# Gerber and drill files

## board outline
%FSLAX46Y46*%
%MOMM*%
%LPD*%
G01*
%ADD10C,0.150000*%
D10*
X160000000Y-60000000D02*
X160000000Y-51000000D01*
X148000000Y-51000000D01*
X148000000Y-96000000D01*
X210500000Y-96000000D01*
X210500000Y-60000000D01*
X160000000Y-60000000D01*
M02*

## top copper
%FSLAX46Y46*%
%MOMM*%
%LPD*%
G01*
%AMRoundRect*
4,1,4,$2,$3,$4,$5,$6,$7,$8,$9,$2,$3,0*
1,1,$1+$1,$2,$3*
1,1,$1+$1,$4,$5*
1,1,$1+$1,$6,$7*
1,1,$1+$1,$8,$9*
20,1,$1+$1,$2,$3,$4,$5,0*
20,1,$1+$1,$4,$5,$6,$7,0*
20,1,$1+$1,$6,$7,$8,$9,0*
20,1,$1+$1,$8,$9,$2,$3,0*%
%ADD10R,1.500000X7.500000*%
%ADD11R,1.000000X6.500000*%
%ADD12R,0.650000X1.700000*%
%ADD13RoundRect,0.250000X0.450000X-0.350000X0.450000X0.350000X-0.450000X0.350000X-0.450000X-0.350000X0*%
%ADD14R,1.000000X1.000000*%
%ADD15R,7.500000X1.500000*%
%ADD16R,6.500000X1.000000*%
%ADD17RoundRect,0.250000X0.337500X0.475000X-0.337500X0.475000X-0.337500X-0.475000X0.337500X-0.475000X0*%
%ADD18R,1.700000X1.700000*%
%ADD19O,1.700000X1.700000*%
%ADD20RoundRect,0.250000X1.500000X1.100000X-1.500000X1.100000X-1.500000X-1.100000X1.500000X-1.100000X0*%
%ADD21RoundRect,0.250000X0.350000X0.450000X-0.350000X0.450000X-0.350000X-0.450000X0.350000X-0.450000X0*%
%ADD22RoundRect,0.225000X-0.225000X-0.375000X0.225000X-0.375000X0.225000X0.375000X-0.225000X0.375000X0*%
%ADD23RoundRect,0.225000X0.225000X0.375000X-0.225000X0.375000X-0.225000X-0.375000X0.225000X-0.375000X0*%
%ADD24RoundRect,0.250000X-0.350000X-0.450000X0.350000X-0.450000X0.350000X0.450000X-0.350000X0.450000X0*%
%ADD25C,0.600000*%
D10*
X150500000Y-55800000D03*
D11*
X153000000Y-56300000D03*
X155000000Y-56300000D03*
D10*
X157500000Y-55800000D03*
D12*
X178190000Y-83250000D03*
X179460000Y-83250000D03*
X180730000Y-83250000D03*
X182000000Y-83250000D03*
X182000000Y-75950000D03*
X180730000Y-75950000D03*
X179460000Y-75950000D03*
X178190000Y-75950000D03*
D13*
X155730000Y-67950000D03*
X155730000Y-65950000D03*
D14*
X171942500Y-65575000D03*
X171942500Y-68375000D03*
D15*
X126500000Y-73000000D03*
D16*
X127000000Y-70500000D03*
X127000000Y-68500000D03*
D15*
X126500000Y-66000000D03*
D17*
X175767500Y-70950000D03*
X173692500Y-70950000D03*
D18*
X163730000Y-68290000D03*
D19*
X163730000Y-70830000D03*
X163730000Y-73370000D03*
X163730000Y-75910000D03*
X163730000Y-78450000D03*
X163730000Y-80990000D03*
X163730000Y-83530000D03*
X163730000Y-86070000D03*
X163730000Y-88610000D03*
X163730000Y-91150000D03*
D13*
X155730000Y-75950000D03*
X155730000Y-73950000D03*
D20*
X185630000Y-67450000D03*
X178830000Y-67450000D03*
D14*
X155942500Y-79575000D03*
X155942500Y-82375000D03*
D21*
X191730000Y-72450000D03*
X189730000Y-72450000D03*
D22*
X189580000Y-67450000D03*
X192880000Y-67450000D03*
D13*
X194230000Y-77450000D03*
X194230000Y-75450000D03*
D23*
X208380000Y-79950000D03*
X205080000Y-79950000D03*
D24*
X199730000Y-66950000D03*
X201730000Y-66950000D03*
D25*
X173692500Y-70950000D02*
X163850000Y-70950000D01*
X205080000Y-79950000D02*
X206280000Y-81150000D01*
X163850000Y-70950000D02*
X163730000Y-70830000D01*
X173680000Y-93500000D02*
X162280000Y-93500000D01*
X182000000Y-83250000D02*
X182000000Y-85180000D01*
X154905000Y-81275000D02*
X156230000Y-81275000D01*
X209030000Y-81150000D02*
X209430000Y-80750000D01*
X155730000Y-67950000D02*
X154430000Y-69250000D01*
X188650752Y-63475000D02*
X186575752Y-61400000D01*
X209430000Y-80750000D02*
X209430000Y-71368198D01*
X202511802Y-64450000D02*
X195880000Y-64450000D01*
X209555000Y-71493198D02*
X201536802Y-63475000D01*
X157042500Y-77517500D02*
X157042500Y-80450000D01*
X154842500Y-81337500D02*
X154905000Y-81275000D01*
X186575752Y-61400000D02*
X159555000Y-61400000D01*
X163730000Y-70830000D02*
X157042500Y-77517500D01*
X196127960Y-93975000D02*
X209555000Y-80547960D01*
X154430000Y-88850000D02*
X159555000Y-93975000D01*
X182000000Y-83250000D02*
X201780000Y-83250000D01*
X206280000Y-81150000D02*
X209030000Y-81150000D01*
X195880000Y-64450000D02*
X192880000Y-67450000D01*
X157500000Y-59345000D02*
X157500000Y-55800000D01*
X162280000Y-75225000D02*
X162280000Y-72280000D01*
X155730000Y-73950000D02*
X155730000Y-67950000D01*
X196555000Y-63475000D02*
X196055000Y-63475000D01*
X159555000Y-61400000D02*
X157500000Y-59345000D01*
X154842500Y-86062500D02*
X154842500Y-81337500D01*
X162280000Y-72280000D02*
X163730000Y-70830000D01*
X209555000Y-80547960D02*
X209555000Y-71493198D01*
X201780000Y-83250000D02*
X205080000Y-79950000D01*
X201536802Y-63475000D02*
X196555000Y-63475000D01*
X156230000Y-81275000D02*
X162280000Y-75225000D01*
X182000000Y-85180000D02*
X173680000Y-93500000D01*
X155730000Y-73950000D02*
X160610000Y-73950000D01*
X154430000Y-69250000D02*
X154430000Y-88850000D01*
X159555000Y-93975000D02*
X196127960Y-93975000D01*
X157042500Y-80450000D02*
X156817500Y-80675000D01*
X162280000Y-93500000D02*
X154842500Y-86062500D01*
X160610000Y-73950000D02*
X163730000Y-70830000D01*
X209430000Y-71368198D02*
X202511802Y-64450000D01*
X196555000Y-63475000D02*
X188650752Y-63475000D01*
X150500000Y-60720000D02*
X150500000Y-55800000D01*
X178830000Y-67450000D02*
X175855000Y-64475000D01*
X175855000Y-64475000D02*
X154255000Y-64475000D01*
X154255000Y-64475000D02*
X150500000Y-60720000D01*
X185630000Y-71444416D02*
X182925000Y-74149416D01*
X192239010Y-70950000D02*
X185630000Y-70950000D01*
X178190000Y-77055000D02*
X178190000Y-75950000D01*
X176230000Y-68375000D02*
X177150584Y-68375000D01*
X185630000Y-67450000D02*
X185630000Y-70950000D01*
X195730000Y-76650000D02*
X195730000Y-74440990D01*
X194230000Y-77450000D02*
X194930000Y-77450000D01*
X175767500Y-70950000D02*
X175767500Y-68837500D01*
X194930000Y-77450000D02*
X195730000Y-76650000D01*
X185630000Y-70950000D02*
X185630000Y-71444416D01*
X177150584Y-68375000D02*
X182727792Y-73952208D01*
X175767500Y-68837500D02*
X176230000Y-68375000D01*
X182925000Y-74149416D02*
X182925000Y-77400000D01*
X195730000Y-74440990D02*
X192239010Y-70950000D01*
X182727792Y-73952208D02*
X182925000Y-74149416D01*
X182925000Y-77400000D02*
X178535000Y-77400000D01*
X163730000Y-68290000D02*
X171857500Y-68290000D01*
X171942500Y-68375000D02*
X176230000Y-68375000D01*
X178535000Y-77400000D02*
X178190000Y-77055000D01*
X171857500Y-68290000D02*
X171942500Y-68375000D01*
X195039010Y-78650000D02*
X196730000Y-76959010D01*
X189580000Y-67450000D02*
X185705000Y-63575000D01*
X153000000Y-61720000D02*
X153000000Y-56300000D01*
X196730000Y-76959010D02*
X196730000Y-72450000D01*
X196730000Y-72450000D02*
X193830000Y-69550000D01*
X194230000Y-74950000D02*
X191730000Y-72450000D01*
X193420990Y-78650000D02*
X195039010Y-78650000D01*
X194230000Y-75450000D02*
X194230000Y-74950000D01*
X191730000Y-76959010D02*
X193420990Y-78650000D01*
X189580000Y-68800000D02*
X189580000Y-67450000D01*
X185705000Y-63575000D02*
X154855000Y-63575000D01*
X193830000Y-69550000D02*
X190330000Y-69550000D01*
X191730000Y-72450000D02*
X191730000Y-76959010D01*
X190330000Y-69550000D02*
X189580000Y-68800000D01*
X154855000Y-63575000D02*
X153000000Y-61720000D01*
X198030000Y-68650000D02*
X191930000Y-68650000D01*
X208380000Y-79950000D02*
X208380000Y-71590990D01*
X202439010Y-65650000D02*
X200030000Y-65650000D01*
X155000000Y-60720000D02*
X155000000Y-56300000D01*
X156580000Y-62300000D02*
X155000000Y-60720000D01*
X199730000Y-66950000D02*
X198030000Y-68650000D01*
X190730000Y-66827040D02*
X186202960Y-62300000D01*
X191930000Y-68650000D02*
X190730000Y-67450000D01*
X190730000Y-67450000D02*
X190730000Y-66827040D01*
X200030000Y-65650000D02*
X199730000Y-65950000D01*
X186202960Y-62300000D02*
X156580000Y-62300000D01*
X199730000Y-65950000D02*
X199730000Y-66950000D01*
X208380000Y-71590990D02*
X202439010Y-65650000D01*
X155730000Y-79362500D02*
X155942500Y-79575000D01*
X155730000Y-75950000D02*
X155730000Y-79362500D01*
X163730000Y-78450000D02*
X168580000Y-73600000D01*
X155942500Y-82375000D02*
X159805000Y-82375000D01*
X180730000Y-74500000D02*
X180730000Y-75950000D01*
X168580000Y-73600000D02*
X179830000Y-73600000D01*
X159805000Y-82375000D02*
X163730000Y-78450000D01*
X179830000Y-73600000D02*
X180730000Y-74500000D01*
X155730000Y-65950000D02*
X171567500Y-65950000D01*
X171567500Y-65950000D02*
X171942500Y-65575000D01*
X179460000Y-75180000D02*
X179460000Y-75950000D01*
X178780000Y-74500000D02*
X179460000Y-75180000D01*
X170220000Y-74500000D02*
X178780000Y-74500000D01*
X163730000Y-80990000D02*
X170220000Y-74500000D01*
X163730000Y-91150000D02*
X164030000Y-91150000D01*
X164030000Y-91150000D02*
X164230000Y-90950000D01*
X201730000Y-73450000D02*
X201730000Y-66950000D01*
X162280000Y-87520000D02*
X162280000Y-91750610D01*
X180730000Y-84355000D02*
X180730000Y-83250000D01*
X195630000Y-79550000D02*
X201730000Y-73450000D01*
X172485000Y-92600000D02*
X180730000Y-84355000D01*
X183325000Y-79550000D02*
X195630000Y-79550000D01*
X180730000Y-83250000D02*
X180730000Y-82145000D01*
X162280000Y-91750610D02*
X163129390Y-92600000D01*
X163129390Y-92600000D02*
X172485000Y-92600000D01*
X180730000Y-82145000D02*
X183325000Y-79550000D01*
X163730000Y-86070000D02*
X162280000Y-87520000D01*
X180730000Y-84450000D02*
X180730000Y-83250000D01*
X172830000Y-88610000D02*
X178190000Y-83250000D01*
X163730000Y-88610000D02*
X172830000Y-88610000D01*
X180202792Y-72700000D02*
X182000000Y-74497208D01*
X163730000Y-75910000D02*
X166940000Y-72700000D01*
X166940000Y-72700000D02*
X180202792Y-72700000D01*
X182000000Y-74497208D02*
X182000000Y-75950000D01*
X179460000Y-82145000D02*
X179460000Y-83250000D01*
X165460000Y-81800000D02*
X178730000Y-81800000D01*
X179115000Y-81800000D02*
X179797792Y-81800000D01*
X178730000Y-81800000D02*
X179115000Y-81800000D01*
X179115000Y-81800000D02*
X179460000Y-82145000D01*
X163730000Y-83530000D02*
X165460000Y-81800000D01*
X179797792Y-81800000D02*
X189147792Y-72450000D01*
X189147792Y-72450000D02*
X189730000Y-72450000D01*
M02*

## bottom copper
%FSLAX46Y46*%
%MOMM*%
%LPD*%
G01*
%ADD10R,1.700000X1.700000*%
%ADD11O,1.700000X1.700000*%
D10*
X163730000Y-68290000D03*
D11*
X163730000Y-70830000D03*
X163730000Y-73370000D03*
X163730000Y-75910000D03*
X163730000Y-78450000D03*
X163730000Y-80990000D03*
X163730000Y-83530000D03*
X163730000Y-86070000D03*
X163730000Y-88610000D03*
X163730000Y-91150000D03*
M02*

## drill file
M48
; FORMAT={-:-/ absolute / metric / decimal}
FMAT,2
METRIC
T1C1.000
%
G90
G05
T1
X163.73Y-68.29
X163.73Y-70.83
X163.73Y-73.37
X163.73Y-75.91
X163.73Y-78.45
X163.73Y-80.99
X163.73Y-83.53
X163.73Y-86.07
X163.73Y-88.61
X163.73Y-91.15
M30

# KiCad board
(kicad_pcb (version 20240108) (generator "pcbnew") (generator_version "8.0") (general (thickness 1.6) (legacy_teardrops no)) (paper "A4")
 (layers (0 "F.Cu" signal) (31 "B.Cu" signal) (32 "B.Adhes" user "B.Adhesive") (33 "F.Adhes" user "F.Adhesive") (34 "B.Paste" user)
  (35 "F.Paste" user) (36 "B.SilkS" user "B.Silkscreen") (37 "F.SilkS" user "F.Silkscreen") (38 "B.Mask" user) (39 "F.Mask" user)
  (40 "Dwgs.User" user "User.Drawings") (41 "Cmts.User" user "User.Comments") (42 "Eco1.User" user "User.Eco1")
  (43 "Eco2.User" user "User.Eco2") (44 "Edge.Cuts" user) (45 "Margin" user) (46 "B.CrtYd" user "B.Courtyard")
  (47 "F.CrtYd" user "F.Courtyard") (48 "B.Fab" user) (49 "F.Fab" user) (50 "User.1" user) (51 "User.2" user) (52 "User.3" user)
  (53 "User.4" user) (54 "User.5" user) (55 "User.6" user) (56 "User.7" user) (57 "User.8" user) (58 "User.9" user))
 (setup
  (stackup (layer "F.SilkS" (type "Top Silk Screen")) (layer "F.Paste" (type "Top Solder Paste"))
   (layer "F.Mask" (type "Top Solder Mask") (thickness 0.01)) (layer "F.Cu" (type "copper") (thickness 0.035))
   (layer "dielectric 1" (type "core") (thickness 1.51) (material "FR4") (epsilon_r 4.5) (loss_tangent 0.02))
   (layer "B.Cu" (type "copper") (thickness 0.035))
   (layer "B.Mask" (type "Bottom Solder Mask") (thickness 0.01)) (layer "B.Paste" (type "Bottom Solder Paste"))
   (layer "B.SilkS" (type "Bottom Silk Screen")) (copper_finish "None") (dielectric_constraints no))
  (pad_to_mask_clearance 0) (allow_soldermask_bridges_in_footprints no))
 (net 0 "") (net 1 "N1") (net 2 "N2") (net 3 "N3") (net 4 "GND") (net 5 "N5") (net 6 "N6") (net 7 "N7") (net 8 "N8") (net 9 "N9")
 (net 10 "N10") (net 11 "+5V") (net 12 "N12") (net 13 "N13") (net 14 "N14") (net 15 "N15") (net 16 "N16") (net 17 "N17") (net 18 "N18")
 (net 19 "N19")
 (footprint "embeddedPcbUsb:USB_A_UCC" (layer "F.Cu") (at 154 56 -90)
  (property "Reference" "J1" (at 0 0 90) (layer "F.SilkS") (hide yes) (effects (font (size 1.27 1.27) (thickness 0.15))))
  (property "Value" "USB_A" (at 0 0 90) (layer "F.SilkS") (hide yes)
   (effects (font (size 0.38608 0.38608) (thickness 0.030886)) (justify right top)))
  (pad "1" smd rect (at -0.2 3.5 270) (size 7.5 1.5) (layers "F.Cu" "F.Paste" "F.Mask") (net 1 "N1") (solder_mask_margin 0.1016))
  (pad "2" smd rect (at 0.3 1 270) (size 6.5 1) (layers "F.Cu" "F.Paste" "F.Mask") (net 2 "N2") (solder_mask_margin 0.1016))
  (pad "3" smd rect (at 0.3 -1 270) (size 6.5 1) (layers "F.Cu" "F.Paste" "F.Mask") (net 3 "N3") (solder_mask_margin 0.1016))
  (pad "4" smd rect (at -0.2 -3.5 270) (size 7.5 1.5) (layers "F.Cu" "F.Paste" "F.Mask") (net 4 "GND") (solder_mask_margin 0.1016)))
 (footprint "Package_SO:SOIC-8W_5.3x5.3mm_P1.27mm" (layer "F.Cu") (at 180.095 79.6 90)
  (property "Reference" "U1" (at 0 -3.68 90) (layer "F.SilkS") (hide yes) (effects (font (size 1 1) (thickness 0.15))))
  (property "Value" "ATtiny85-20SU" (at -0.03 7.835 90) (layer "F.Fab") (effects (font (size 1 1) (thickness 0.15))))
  (pad "1" smd rect (at -3.65 -1.905 90) (size 1.7 0.65) (layers "F.Cu" "F.Paste" "F.Mask") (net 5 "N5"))
  (pad "2" smd rect (at -3.65 -0.635 90) (size 1.7 0.65) (layers "F.Cu" "F.Paste" "F.Mask") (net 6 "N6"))
  (pad "3" smd rect (at -3.65 0.635 90) (size 1.7 0.65) (layers "F.Cu" "F.Paste" "F.Mask") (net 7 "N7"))
  (pad "4" smd rect (at -3.65 1.905 90) (size 1.7 0.65) (layers "F.Cu" "F.Paste" "F.Mask") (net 4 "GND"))
  (pad "5" smd rect (at 3.65 1.905 90) (size 1.7 0.65) (layers "F.Cu" "F.Paste" "F.Mask") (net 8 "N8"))
  (pad "6" smd rect (at 3.65 0.635 90) (size 1.7 0.65) (layers "F.Cu" "F.Paste" "F.Mask") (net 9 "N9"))
  (pad "7" smd rect (at 3.65 -0.635 90) (size 1.7 0.65) (layers "F.Cu" "F.Paste" "F.Mask") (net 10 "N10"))
  (pad "8" smd rect (at 3.65 -1.905 90) (size 1.7 0.65) (layers "F.Cu" "F.Paste" "F.Mask") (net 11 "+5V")))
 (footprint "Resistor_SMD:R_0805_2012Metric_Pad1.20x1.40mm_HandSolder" (layer "F.Cu") (at 155.73 66.95 90)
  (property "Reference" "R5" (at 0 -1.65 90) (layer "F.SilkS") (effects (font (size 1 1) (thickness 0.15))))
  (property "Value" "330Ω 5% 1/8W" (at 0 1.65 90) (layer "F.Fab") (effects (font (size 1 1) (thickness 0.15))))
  (pad "1" smd roundrect (at -1 0 90) (size 1.2 1.4) (layers "F.Cu" "F.Paste" "F.Mask") (roundrect_rratio 0.208333) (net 4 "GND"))
  (pad "2" smd roundrect (at 1 0 90) (size 1.2 1.4) (layers "F.Cu" "F.Paste" "F.Mask") (roundrect_rratio 0.208333) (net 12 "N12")))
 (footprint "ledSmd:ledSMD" (layer "F.Cu") (at 171.9425 67.375 -90)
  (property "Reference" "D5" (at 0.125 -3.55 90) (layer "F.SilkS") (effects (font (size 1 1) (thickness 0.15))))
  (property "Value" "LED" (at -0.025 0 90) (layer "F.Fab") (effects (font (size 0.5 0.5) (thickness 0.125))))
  (pad "1" smd rect (at -1.8 0 270) (size 1 1) (layers "F.Cu" "F.Paste" "F.Mask") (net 12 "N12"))
  (pad "2" smd rect (at 1 0 270) (size 1 1) (layers "F.Cu" "F.Paste" "F.Mask") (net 11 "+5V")))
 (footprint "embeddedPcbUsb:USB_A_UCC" (layer "F.Cu") (at 126.7 69.5)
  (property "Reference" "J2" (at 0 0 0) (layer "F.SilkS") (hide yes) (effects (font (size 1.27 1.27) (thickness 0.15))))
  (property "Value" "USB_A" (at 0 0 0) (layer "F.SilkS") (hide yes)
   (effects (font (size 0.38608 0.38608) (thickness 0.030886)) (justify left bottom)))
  (pad "1" smd rect (at -0.2 3.5) (size 7.5 1.5) (layers "F.Cu" "F.Paste" "F.Mask") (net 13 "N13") (solder_mask_margin 0.1016))
  (pad "2" smd rect (at 0.3 1) (size 6.5 1) (layers "F.Cu" "F.Paste" "F.Mask") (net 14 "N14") (solder_mask_margin 0.1016))
  (pad "3" smd rect (at 0.3 -1) (size 6.5 1) (layers "F.Cu" "F.Paste" "F.Mask") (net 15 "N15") (solder_mask_margin 0.1016))
  (pad "4" smd rect (at -0.2 -3.5) (size 7.5 1.5) (layers "F.Cu" "F.Paste" "F.Mask") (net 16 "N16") (solder_mask_margin 0.1016)))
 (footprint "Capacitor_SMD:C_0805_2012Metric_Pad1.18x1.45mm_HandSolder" (layer "F.Cu") (at 174.73 70.95 180)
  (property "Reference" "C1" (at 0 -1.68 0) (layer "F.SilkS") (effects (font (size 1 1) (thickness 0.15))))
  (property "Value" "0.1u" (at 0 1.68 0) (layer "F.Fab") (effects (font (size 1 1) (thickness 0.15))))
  (pad "1" smd roundrect (at -1.0375 0 180) (size 1.175 1.45) (layers "F.Cu" "F.Paste" "F.Mask") (roundrect_rratio 0.212766) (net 11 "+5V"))
  (pad "2" smd roundrect (at 1.0375 0 180) (size 1.175 1.45) (layers "F.Cu" "F.Paste" "F.Mask") (roundrect_rratio 0.212766) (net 4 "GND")))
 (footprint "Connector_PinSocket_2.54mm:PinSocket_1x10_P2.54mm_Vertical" (layer "F.Cu") (at 163.73 68.29)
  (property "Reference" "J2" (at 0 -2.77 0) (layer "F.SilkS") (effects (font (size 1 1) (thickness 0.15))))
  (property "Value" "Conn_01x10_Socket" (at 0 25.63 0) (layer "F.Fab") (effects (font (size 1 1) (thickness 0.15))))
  (pad "1" thru_hole rect (at 0 0) (size 1.7 1.7) (drill 1) (layers "*.Cu" "*.Mask") (remove_unused_layers no) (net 11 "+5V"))
  (pad "2" thru_hole oval (at 0 2.54) (size 1.7 1.7) (drill 1) (layers "*.Cu" "*.Mask") (remove_unused_layers no) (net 4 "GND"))
  (pad "3" thru_hole oval (at 0 5.08) (size 1.7 1.7) (drill 1) (layers "*.Cu" "*.Mask") (remove_unused_layers no) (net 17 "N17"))
  (pad "4" thru_hole oval (at 0 7.62) (size 1.7 1.7) (drill 1) (layers "*.Cu" "*.Mask") (remove_unused_layers no) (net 8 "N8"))
  (pad "5" thru_hole oval (at 0 10.16) (size 1.7 1.7) (drill 1) (layers "*.Cu" "*.Mask") (remove_unused_layers no) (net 9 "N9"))
  (pad "6" thru_hole oval (at 0 12.7) (size 1.7 1.7) (drill 1) (layers "*.Cu" "*.Mask") (remove_unused_layers no) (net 10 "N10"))
  (pad "7" thru_hole oval (at 0 15.24) (size 1.7 1.7) (drill 1) (layers "*.Cu" "*.Mask") (remove_unused_layers no) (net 6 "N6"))
  (pad "8" thru_hole oval (at 0 17.78) (size 1.7 1.7) (drill 1) (layers "*.Cu" "*.Mask") (remove_unused_layers no) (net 7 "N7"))
  (pad "9" thru_hole oval (at 0 20.32) (size 1.7 1.7) (drill 1) (layers "*.Cu" "*.Mask") (remove_unused_layers no) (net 5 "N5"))
  (pad "10" thru_hole oval (at 0 22.86) (size 1.7 1.7) (drill 1) (layers "*.Cu" "*.Mask") (remove_unused_layers no) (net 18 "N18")))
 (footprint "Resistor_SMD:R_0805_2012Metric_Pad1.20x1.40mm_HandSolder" (layer "F.Cu") (at 155.73 74.95 90)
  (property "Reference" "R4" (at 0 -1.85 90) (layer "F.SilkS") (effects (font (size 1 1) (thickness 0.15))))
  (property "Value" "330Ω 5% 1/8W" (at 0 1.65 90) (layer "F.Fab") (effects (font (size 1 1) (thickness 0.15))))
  (pad "1" smd roundrect (at -1 0 90) (size 1.2 1.4) (layers "F.Cu" "F.Paste" "F.Mask") (roundrect_rratio 0.208333) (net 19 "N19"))
  (pad "2" smd roundrect (at 1 0 90) (size 1.2 1.4) (layers "F.Cu" "F.Paste" "F.Mask") (roundrect_rratio 0.208333) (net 4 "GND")))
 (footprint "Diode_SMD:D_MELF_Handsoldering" (layer "F.Cu") (at 182.23 67.45 180)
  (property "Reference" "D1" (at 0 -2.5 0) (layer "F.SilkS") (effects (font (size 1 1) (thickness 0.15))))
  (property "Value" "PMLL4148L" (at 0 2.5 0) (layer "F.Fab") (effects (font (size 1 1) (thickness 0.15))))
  (pad "1" smd roundrect (at -3.4 0 180) (size 3.5 2.7) (layers "F.Cu" "F.Paste" "F.Mask") (roundrect_rratio 0.0925925926) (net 11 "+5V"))
  (pad "2" smd roundrect (at 3.4 0 180) (size 3.5 2.7) (layers "F.Cu" "F.Paste" "F.Mask") (roundrect_rratio 0.0925925926) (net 1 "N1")))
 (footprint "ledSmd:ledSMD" (layer "F.Cu") (at 155.9425 81.375 -90)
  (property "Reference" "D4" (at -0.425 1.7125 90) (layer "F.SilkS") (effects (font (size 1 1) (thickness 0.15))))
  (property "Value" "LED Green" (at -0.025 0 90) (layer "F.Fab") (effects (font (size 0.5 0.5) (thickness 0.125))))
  (pad "1" smd rect (at -1.8 0 270) (size 1 1) (layers "F.Cu" "F.Paste" "F.Mask") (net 19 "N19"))
  (pad "2" smd rect (at 1 0 270) (size 1 1) (layers "F.Cu" "F.Paste" "F.Mask") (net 9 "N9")))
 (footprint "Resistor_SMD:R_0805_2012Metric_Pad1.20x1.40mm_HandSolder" (layer "F.Cu") (at 190.73 72.45 180)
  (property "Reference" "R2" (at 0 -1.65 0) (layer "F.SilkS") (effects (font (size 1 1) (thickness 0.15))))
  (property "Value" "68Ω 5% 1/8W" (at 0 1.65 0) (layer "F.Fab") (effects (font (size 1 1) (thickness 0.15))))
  (pad "1" smd roundrect (at -1 0 180) (size 1.2 1.4) (layers "F.Cu" "F.Paste" "F.Mask") (roundrect_rratio 0.208333) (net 2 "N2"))
  (pad "2" smd roundrect (at 1 0 180) (size 1.2 1.4) (layers "F.Cu" "F.Paste" "F.Mask") (roundrect_rratio 0.208333) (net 6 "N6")))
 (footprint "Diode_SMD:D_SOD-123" (layer "F.Cu") (at 191.23 67.45)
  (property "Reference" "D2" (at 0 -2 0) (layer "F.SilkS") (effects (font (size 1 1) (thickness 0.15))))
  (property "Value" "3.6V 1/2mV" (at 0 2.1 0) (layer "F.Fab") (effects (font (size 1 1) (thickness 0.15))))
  (pad "1" smd roundrect (at -1.65 0) (size 0.9 1.2) (layers "F.Cu" "F.Paste" "F.Mask") (roundrect_rratio 0.25) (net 2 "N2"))
  (pad "2" smd roundrect (at 1.65 0) (size 0.9 1.2) (layers "F.Cu" "F.Paste" "F.Mask") (roundrect_rratio 0.25) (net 4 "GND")))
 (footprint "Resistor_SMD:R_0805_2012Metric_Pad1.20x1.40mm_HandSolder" (layer "F.Cu") (at 194.23 76.45 90)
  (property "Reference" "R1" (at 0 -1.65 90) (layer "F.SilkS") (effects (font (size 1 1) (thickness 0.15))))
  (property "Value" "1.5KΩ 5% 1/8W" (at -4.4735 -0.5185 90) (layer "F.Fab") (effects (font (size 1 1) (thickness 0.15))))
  (pad "1" smd roundrect (at -1 0 90) (size 1.2 1.4) (layers "F.Cu" "F.Paste" "F.Mask") (roundrect_rratio 0.208333) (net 11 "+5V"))
  (pad "2" smd roundrect (at 1 0 90) (size 1.2 1.4) (layers "F.Cu" "F.Paste" "F.Mask") (roundrect_rratio 0.208333) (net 2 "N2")))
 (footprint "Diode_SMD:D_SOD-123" (layer "F.Cu") (at 206.73 79.95 180)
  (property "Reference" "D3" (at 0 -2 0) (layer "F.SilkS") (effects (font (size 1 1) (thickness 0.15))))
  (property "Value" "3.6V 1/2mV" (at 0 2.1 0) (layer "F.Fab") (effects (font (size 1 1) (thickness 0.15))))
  (pad "1" smd roundrect (at -1.65 0 180) (size 0.9 1.2) (layers "F.Cu" "F.Paste" "F.Mask") (roundrect_rratio 0.25) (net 3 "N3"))
  (pad "2" smd roundrect (at 1.65 0 180) (size 0.9 1.2) (layers "F.Cu" "F.Paste" "F.Mask") (roundrect_rratio 0.25) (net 4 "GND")))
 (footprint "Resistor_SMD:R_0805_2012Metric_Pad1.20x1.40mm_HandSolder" (layer "F.Cu") (at 200.73 66.95)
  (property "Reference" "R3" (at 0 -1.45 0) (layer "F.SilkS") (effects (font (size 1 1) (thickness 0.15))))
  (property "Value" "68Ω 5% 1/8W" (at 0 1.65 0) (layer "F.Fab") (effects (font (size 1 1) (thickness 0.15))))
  (pad "1" smd roundrect (at -1 0) (size 1.2 1.4) (layers "F.Cu" "F.Paste" "F.Mask") (roundrect_rratio 0.208333) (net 3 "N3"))
  (pad "2" smd roundrect (at 1 0) (size 1.2 1.4) (layers "F.Cu" "F.Paste" "F.Mask") (roundrect_rratio 0.208333) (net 7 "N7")))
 (gr_poly
  (pts (xy 160 60) (xy 160 51) (xy 148 51) (xy 148 96) (xy 210.5 96) (xy 210.5 60)) (stroke (width 0.15) (type solid)) (fill none)
  (layer "Edge.Cuts"))
 (segment (start 173.6925 70.95) (end 163.85 70.95) (width 0.6) (layer "F.Cu") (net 4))
 (segment (start 205.08 79.95) (end 206.28 81.15) (width 0.6) (layer "F.Cu") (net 4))
 (segment (start 163.85 70.95) (end 163.73 70.83) (width 0.6) (layer "F.Cu") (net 4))
 (segment (start 173.68 93.5) (end 162.28 93.5) (width 0.6) (layer "F.Cu") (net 4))
 (segment (start 182 83.25) (end 182 85.18) (width 0.6) (layer "F.Cu") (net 4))
 (segment (start 154.905 81.275) (end 156.23 81.275) (width 0.6) (layer "F.Cu") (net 4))
 (segment (start 209.03 81.15) (end 209.43 80.75) (width 0.6) (layer "F.Cu") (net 4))
 (segment (start 155.73 67.95) (end 154.43 69.25) (width 0.6) (layer "F.Cu") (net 4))
 (segment (start 188.650752 63.475) (end 186.575752 61.4) (width 0.6) (layer "F.Cu") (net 4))
 (segment (start 209.43 80.75) (end 209.43 71.368198) (width 0.6) (layer "F.Cu") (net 4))
 (segment (start 202.511802 64.45) (end 195.88 64.45) (width 0.6) (layer "F.Cu") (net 4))
 (segment (start 209.555 71.493198) (end 201.536802 63.475) (width 0.6) (layer "F.Cu") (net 4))
 (segment (start 157.0425 77.5175) (end 157.0425 80.45) (width 0.6) (layer "F.Cu") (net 4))
 (segment (start 154.8425 81.3375) (end 154.905 81.275) (width 0.6) (layer "F.Cu") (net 4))
 (segment (start 186.575752 61.4) (end 159.555 61.4) (width 0.6) (layer "F.Cu") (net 4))
 (segment (start 163.73 70.83) (end 157.0425 77.5175) (width 0.6) (layer "F.Cu") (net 4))
 (segment (start 196.12796 93.975) (end 209.555 80.54796) (width 0.6) (layer "F.Cu") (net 4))
 (segment (start 154.43 88.85) (end 159.555 93.975) (width 0.6) (layer "F.Cu") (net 4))
 (segment (start 182 83.25) (end 201.78 83.25) (width 0.6) (layer "F.Cu") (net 4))
 (segment (start 206.28 81.15) (end 209.03 81.15) (width 0.6) (layer "F.Cu") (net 4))
 (segment (start 195.88 64.45) (end 192.88 67.45) (width 0.6) (layer "F.Cu") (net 4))
 (segment (start 157.5 59.345) (end 157.5 55.8) (width 0.6) (layer "F.Cu") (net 4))
 (segment (start 162.28 75.225) (end 162.28 72.28) (width 0.6) (layer "F.Cu") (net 4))
 (segment (start 155.73 73.95) (end 155.73 67.95) (width 0.6) (layer "F.Cu") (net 4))
 (segment (start 196.555 63.475) (end 196.055 63.475) (width 0.6) (layer "F.Cu") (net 4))
 (segment (start 159.555 61.4) (end 157.5 59.345) (width 0.6) (layer "F.Cu") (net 4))
 (segment (start 154.8425 86.0625) (end 154.8425 81.3375) (width 0.6) (layer "F.Cu") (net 4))
 (segment (start 162.28 72.28) (end 163.73 70.83) (width 0.6) (layer "F.Cu") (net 4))
 (segment (start 209.555 80.54796) (end 209.555 71.493198) (width 0.6) (layer "F.Cu") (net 4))
 (segment (start 201.78 83.25) (end 205.08 79.95) (width 0.6) (layer "F.Cu") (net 4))
 (segment (start 201.536802 63.475) (end 196.555 63.475) (width 0.6) (layer "F.Cu") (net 4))
 (segment (start 156.23 81.275) (end 162.28 75.225) (width 0.6) (layer "F.Cu") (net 4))
 (segment (start 182 85.18) (end 173.68 93.5) (width 0.6) (layer "F.Cu") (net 4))
 (segment (start 155.73 73.95) (end 160.61 73.95) (width 0.6) (layer "F.Cu") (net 4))
 (segment (start 154.43 69.25) (end 154.43 88.85) (width 0.6) (layer "F.Cu") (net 4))
 (segment (start 159.555 93.975) (end 196.12796 93.975) (width 0.6) (layer "F.Cu") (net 4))
 (segment (start 157.0425 80.45) (end 156.8175 80.675) (width 0.6) (layer "F.Cu") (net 4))
 (segment (start 162.28 93.5) (end 154.8425 86.0625) (width 0.6) (layer "F.Cu") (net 4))
 (segment (start 160.61 73.95) (end 163.73 70.83) (width 0.6) (layer "F.Cu") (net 4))
 (segment (start 209.43 71.368198) (end 202.511802 64.45) (width 0.6) (layer "F.Cu") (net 4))
 (segment (start 196.555 63.475) (end 188.650752 63.475) (width 0.6) (layer "F.Cu") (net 4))
 (segment (start 150.5 60.72) (end 150.5 55.8) (width 0.6) (layer "F.Cu") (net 1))
 (segment (start 178.83 67.45) (end 175.855 64.475) (width 0.6) (layer "F.Cu") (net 1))
 (segment (start 175.855 64.475) (end 154.255 64.475) (width 0.6) (layer "F.Cu") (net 1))
 (segment (start 154.255 64.475) (end 150.5 60.72) (width 0.6) (layer "F.Cu") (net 1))
 (segment (start 185.63 71.444416) (end 182.925 74.149416) (width 0.6) (layer "F.Cu") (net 11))
 (segment (start 192.23901 70.95) (end 185.63 70.95) (width 0.6) (layer "F.Cu") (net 11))
 (segment (start 178.19 77.055) (end 178.19 75.95) (width 0.6) (layer "F.Cu") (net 11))
 (segment (start 176.23 68.375) (end 177.150584 68.375) (width 0.6) (layer "F.Cu") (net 11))
 (segment (start 185.63 67.45) (end 185.63 70.95) (width 0.6) (layer "F.Cu") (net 11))
 (segment (start 195.73 76.65) (end 195.73 74.44099) (width 0.6) (layer "F.Cu") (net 11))
 (segment (start 194.23 77.45) (end 194.93 77.45) (width 0.6) (layer "F.Cu") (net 11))
 (segment (start 175.7675 70.95) (end 175.7675 68.8375) (width 0.6) (layer "F.Cu") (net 11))
 (segment (start 194.93 77.45) (end 195.73 76.65) (width 0.6) (layer "F.Cu") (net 11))
 (segment (start 185.63 70.95) (end 185.63 71.444416) (width 0.6) (layer "F.Cu") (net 11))
 (segment (start 177.150584 68.375) (end 182.727792 73.952208) (width 0.6) (layer "F.Cu") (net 11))
 (segment (start 175.7675 68.8375) (end 176.23 68.375) (width 0.6) (layer "F.Cu") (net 11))
 (segment (start 182.925 74.149416) (end 182.925 77.4) (width 0.6) (layer "F.Cu") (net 11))
 (segment (start 195.73 74.44099) (end 192.23901 70.95) (width 0.6) (layer "F.Cu") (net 11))
 (segment (start 182.727792 73.952208) (end 182.925 74.149416) (width 0.6) (layer "F.Cu") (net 11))
 (segment (start 182.925 77.4) (end 178.535 77.4) (width 0.6) (layer "F.Cu") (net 11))
 (segment (start 163.73 68.29) (end 171.8575 68.29) (width 0.6) (layer "F.Cu") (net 11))
 (segment (start 171.9425 68.375) (end 176.23 68.375) (width 0.6) (layer "F.Cu") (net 11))
 (segment (start 178.535 77.4) (end 178.19 77.055) (width 0.6) (layer "F.Cu") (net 11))
 (segment (start 171.8575 68.29) (end 171.9425 68.375) (width 0.6) (layer "F.Cu") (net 11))
 (segment (start 195.03901 78.65) (end 196.73 76.95901) (width 0.6) (layer "F.Cu") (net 2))
 (segment (start 189.58 67.45) (end 185.705 63.575) (width 0.6) (layer "F.Cu") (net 2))
 (segment (start 153 61.72) (end 153 56.3) (width 0.6) (layer "F.Cu") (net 2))
 (segment (start 196.73 76.95901) (end 196.73 72.45) (width 0.6) (layer "F.Cu") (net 2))
 (segment (start 196.73 72.45) (end 193.83 69.55) (width 0.6) (layer "F.Cu") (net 2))
 (segment (start 194.23 74.95) (end 191.73 72.45) (width 0.6) (layer "F.Cu") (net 2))
 (segment (start 193.42099 78.65) (end 195.03901 78.65) (width 0.6) (layer "F.Cu") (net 2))
 (segment (start 194.23 75.45) (end 194.23 74.95) (width 0.6) (layer "F.Cu") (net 2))
 (segment (start 191.73 76.95901) (end 193.42099 78.65) (width 0.6) (layer "F.Cu") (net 2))
 (segment (start 189.58 68.8) (end 189.58 67.45) (width 0.6) (layer "F.Cu") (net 2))
 (segment (start 185.705 63.575) (end 154.855 63.575) (width 0.6) (layer "F.Cu") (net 2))
 (segment (start 193.83 69.55) (end 190.33 69.55) (width 0.6) (layer "F.Cu") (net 2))
 (segment (start 191.73 72.45) (end 191.73 76.95901) (width 0.6) (layer "F.Cu") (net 2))
 (segment (start 190.33 69.55) (end 189.58 68.8) (width 0.6) (layer "F.Cu") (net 2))
 (segment (start 154.855 63.575) (end 153 61.72) (width 0.6) (layer "F.Cu") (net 2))
 (segment (start 198.03 68.65) (end 191.93 68.65) (width 0.6) (layer "F.Cu") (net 3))
 (segment (start 208.38 79.95) (end 208.38 71.59099) (width 0.6) (layer "F.Cu") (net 3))
 (segment (start 202.43901 65.65) (end 200.03 65.65) (width 0.6) (layer "F.Cu") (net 3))
 (segment (start 155 60.72) (end 155 56.3) (width 0.6) (layer "F.Cu") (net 3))
 (segment (start 156.58 62.3) (end 155 60.72) (width 0.6) (layer "F.Cu") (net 3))
 (segment (start 199.73 66.95) (end 198.03 68.65) (width 0.6) (layer "F.Cu") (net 3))
 (segment (start 190.73 66.82704) (end 186.20296 62.3) (width 0.6) (layer "F.Cu") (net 3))
 (segment (start 191.93 68.65) (end 190.73 67.45) (width 0.6) (layer "F.Cu") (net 3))
 (segment (start 190.73 67.45) (end 190.73 66.82704) (width 0.6) (layer "F.Cu") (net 3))
 (segment (start 200.03 65.65) (end 199.73 65.95) (width 0.6) (layer "F.Cu") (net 3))
 (segment (start 186.20296 62.3) (end 156.58 62.3) (width 0.6) (layer "F.Cu") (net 3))
 (segment (start 199.73 65.95) (end 199.73 66.95) (width 0.6) (layer "F.Cu") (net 3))
 (segment (start 208.38 71.59099) (end 202.43901 65.65) (width 0.6) (layer "F.Cu") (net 3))
 (segment (start 155.73 79.3625) (end 155.9425 79.575) (width 0.6) (layer "F.Cu") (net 19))
 (segment (start 155.73 75.95) (end 155.73 79.3625) (width 0.6) (layer "F.Cu") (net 19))
 (segment (start 163.73 78.45) (end 168.58 73.6) (width 0.6) (layer "F.Cu") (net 9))
 (segment (start 155.9425 82.375) (end 159.805 82.375) (width 0.6) (layer "F.Cu") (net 9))
 (segment (start 180.73 74.5) (end 180.73 75.95) (width 0.6) (layer "F.Cu") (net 9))
 (segment (start 168.58 73.6) (end 179.83 73.6) (width 0.6) (layer "F.Cu") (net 9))
 (segment (start 159.805 82.375) (end 163.73 78.45) (width 0.6) (layer "F.Cu") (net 9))
 (segment (start 179.83 73.6) (end 180.73 74.5) (width 0.6) (layer "F.Cu") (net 9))
 (segment (start 155.73 65.95) (end 171.5675 65.95) (width 0.6) (layer "F.Cu") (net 12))
 (segment (start 171.5675 65.95) (end 171.9425 65.575) (width 0.6) (layer "F.Cu") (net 12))
 (segment (start 179.46 75.18) (end 179.46 75.95) (width 0.6) (layer "F.Cu") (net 10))
 (segment (start 178.78 74.5) (end 179.46 75.18) (width 0.6) (layer "F.Cu") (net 10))
 (segment (start 170.22 74.5) (end 178.78 74.5) (width 0.6) (layer "F.Cu") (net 10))
 (segment (start 163.73 80.99) (end 170.22 74.5) (width 0.6) (layer "F.Cu") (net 10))
 (segment (start 163.73 91.15) (end 164.03 91.15) (width 0.6) (layer "F.Cu") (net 18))
 (segment (start 164.03 91.15) (end 164.23 90.95) (width 0.6) (layer "F.Cu") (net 18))
 (segment (start 201.73 73.45) (end 201.73 66.95) (width 0.6) (layer "F.Cu") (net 7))
 (segment (start 162.28 87.52) (end 162.28 91.75061) (width 0.6) (layer "F.Cu") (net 7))
 (segment (start 180.73 84.355) (end 180.73 83.25) (width 0.6) (layer "F.Cu") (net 7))
 (segment (start 195.63 79.55) (end 201.73 73.45) (width 0.6) (layer "F.Cu") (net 7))
 (segment (start 172.485 92.6) (end 180.73 84.355) (width 0.6) (layer "F.Cu") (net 7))
 (segment (start 183.325 79.55) (end 195.63 79.55) (width 0.6) (layer "F.Cu") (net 7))
 (segment (start 180.73 83.25) (end 180.73 82.145) (width 0.6) (layer "F.Cu") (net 7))
 (segment (start 162.28 91.75061) (end 163.12939 92.6) (width 0.6) (layer "F.Cu") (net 7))
 (segment (start 163.12939 92.6) (end 172.485 92.6) (width 0.6) (layer "F.Cu") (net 7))
 (segment (start 180.73 82.145) (end 183.325 79.55) (width 0.6) (layer "F.Cu") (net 7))
 (segment (start 163.73 86.07) (end 162.28 87.52) (width 0.6) (layer "F.Cu") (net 7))
 (segment (start 180.73 84.45) (end 180.73 83.25) (width 0.6) (layer "F.Cu") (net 7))
 (segment (start 172.83 88.61) (end 178.19 83.25) (width 0.6) (layer "F.Cu") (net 5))
 (segment (start 163.73 88.61) (end 172.83 88.61) (width 0.6) (layer "F.Cu") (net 5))
 (segment (start 180.202792 72.7) (end 182 74.497208) (width 0.6) (layer "F.Cu") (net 8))
 (segment (start 163.73 75.91) (end 166.94 72.7) (width 0.6) (layer "F.Cu") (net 8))
 (segment (start 166.94 72.7) (end 180.202792 72.7) (width 0.6) (layer "F.Cu") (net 8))
 (segment (start 182 74.497208) (end 182 75.95) (width 0.6) (layer "F.Cu") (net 8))
 (segment (start 179.46 82.145) (end 179.46 83.25) (width 0.6) (layer "F.Cu") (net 6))
 (segment (start 165.46 81.8) (end 178.73 81.8) (width 0.6) (layer "F.Cu") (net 6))
 (segment (start 179.115 81.8) (end 179.797792 81.8) (width 0.6) (layer "F.Cu") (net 6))
 (segment (start 178.73 81.8) (end 179.115 81.8) (width 0.6) (layer "F.Cu") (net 6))
 (segment (start 179.115 81.8) (end 179.46 82.145) (width 0.6) (layer "F.Cu") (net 6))
 (segment (start 163.73 83.53) (end 165.46 81.8) (width 0.6) (layer "F.Cu") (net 6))
 (segment (start 179.797792 81.8) (end 189.147792 72.45) (width 0.6) (layer "F.Cu") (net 6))
 (segment (start 189.147792 72.45) (end 189.73 72.45) (width 0.6) (layer "F.Cu") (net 6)))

